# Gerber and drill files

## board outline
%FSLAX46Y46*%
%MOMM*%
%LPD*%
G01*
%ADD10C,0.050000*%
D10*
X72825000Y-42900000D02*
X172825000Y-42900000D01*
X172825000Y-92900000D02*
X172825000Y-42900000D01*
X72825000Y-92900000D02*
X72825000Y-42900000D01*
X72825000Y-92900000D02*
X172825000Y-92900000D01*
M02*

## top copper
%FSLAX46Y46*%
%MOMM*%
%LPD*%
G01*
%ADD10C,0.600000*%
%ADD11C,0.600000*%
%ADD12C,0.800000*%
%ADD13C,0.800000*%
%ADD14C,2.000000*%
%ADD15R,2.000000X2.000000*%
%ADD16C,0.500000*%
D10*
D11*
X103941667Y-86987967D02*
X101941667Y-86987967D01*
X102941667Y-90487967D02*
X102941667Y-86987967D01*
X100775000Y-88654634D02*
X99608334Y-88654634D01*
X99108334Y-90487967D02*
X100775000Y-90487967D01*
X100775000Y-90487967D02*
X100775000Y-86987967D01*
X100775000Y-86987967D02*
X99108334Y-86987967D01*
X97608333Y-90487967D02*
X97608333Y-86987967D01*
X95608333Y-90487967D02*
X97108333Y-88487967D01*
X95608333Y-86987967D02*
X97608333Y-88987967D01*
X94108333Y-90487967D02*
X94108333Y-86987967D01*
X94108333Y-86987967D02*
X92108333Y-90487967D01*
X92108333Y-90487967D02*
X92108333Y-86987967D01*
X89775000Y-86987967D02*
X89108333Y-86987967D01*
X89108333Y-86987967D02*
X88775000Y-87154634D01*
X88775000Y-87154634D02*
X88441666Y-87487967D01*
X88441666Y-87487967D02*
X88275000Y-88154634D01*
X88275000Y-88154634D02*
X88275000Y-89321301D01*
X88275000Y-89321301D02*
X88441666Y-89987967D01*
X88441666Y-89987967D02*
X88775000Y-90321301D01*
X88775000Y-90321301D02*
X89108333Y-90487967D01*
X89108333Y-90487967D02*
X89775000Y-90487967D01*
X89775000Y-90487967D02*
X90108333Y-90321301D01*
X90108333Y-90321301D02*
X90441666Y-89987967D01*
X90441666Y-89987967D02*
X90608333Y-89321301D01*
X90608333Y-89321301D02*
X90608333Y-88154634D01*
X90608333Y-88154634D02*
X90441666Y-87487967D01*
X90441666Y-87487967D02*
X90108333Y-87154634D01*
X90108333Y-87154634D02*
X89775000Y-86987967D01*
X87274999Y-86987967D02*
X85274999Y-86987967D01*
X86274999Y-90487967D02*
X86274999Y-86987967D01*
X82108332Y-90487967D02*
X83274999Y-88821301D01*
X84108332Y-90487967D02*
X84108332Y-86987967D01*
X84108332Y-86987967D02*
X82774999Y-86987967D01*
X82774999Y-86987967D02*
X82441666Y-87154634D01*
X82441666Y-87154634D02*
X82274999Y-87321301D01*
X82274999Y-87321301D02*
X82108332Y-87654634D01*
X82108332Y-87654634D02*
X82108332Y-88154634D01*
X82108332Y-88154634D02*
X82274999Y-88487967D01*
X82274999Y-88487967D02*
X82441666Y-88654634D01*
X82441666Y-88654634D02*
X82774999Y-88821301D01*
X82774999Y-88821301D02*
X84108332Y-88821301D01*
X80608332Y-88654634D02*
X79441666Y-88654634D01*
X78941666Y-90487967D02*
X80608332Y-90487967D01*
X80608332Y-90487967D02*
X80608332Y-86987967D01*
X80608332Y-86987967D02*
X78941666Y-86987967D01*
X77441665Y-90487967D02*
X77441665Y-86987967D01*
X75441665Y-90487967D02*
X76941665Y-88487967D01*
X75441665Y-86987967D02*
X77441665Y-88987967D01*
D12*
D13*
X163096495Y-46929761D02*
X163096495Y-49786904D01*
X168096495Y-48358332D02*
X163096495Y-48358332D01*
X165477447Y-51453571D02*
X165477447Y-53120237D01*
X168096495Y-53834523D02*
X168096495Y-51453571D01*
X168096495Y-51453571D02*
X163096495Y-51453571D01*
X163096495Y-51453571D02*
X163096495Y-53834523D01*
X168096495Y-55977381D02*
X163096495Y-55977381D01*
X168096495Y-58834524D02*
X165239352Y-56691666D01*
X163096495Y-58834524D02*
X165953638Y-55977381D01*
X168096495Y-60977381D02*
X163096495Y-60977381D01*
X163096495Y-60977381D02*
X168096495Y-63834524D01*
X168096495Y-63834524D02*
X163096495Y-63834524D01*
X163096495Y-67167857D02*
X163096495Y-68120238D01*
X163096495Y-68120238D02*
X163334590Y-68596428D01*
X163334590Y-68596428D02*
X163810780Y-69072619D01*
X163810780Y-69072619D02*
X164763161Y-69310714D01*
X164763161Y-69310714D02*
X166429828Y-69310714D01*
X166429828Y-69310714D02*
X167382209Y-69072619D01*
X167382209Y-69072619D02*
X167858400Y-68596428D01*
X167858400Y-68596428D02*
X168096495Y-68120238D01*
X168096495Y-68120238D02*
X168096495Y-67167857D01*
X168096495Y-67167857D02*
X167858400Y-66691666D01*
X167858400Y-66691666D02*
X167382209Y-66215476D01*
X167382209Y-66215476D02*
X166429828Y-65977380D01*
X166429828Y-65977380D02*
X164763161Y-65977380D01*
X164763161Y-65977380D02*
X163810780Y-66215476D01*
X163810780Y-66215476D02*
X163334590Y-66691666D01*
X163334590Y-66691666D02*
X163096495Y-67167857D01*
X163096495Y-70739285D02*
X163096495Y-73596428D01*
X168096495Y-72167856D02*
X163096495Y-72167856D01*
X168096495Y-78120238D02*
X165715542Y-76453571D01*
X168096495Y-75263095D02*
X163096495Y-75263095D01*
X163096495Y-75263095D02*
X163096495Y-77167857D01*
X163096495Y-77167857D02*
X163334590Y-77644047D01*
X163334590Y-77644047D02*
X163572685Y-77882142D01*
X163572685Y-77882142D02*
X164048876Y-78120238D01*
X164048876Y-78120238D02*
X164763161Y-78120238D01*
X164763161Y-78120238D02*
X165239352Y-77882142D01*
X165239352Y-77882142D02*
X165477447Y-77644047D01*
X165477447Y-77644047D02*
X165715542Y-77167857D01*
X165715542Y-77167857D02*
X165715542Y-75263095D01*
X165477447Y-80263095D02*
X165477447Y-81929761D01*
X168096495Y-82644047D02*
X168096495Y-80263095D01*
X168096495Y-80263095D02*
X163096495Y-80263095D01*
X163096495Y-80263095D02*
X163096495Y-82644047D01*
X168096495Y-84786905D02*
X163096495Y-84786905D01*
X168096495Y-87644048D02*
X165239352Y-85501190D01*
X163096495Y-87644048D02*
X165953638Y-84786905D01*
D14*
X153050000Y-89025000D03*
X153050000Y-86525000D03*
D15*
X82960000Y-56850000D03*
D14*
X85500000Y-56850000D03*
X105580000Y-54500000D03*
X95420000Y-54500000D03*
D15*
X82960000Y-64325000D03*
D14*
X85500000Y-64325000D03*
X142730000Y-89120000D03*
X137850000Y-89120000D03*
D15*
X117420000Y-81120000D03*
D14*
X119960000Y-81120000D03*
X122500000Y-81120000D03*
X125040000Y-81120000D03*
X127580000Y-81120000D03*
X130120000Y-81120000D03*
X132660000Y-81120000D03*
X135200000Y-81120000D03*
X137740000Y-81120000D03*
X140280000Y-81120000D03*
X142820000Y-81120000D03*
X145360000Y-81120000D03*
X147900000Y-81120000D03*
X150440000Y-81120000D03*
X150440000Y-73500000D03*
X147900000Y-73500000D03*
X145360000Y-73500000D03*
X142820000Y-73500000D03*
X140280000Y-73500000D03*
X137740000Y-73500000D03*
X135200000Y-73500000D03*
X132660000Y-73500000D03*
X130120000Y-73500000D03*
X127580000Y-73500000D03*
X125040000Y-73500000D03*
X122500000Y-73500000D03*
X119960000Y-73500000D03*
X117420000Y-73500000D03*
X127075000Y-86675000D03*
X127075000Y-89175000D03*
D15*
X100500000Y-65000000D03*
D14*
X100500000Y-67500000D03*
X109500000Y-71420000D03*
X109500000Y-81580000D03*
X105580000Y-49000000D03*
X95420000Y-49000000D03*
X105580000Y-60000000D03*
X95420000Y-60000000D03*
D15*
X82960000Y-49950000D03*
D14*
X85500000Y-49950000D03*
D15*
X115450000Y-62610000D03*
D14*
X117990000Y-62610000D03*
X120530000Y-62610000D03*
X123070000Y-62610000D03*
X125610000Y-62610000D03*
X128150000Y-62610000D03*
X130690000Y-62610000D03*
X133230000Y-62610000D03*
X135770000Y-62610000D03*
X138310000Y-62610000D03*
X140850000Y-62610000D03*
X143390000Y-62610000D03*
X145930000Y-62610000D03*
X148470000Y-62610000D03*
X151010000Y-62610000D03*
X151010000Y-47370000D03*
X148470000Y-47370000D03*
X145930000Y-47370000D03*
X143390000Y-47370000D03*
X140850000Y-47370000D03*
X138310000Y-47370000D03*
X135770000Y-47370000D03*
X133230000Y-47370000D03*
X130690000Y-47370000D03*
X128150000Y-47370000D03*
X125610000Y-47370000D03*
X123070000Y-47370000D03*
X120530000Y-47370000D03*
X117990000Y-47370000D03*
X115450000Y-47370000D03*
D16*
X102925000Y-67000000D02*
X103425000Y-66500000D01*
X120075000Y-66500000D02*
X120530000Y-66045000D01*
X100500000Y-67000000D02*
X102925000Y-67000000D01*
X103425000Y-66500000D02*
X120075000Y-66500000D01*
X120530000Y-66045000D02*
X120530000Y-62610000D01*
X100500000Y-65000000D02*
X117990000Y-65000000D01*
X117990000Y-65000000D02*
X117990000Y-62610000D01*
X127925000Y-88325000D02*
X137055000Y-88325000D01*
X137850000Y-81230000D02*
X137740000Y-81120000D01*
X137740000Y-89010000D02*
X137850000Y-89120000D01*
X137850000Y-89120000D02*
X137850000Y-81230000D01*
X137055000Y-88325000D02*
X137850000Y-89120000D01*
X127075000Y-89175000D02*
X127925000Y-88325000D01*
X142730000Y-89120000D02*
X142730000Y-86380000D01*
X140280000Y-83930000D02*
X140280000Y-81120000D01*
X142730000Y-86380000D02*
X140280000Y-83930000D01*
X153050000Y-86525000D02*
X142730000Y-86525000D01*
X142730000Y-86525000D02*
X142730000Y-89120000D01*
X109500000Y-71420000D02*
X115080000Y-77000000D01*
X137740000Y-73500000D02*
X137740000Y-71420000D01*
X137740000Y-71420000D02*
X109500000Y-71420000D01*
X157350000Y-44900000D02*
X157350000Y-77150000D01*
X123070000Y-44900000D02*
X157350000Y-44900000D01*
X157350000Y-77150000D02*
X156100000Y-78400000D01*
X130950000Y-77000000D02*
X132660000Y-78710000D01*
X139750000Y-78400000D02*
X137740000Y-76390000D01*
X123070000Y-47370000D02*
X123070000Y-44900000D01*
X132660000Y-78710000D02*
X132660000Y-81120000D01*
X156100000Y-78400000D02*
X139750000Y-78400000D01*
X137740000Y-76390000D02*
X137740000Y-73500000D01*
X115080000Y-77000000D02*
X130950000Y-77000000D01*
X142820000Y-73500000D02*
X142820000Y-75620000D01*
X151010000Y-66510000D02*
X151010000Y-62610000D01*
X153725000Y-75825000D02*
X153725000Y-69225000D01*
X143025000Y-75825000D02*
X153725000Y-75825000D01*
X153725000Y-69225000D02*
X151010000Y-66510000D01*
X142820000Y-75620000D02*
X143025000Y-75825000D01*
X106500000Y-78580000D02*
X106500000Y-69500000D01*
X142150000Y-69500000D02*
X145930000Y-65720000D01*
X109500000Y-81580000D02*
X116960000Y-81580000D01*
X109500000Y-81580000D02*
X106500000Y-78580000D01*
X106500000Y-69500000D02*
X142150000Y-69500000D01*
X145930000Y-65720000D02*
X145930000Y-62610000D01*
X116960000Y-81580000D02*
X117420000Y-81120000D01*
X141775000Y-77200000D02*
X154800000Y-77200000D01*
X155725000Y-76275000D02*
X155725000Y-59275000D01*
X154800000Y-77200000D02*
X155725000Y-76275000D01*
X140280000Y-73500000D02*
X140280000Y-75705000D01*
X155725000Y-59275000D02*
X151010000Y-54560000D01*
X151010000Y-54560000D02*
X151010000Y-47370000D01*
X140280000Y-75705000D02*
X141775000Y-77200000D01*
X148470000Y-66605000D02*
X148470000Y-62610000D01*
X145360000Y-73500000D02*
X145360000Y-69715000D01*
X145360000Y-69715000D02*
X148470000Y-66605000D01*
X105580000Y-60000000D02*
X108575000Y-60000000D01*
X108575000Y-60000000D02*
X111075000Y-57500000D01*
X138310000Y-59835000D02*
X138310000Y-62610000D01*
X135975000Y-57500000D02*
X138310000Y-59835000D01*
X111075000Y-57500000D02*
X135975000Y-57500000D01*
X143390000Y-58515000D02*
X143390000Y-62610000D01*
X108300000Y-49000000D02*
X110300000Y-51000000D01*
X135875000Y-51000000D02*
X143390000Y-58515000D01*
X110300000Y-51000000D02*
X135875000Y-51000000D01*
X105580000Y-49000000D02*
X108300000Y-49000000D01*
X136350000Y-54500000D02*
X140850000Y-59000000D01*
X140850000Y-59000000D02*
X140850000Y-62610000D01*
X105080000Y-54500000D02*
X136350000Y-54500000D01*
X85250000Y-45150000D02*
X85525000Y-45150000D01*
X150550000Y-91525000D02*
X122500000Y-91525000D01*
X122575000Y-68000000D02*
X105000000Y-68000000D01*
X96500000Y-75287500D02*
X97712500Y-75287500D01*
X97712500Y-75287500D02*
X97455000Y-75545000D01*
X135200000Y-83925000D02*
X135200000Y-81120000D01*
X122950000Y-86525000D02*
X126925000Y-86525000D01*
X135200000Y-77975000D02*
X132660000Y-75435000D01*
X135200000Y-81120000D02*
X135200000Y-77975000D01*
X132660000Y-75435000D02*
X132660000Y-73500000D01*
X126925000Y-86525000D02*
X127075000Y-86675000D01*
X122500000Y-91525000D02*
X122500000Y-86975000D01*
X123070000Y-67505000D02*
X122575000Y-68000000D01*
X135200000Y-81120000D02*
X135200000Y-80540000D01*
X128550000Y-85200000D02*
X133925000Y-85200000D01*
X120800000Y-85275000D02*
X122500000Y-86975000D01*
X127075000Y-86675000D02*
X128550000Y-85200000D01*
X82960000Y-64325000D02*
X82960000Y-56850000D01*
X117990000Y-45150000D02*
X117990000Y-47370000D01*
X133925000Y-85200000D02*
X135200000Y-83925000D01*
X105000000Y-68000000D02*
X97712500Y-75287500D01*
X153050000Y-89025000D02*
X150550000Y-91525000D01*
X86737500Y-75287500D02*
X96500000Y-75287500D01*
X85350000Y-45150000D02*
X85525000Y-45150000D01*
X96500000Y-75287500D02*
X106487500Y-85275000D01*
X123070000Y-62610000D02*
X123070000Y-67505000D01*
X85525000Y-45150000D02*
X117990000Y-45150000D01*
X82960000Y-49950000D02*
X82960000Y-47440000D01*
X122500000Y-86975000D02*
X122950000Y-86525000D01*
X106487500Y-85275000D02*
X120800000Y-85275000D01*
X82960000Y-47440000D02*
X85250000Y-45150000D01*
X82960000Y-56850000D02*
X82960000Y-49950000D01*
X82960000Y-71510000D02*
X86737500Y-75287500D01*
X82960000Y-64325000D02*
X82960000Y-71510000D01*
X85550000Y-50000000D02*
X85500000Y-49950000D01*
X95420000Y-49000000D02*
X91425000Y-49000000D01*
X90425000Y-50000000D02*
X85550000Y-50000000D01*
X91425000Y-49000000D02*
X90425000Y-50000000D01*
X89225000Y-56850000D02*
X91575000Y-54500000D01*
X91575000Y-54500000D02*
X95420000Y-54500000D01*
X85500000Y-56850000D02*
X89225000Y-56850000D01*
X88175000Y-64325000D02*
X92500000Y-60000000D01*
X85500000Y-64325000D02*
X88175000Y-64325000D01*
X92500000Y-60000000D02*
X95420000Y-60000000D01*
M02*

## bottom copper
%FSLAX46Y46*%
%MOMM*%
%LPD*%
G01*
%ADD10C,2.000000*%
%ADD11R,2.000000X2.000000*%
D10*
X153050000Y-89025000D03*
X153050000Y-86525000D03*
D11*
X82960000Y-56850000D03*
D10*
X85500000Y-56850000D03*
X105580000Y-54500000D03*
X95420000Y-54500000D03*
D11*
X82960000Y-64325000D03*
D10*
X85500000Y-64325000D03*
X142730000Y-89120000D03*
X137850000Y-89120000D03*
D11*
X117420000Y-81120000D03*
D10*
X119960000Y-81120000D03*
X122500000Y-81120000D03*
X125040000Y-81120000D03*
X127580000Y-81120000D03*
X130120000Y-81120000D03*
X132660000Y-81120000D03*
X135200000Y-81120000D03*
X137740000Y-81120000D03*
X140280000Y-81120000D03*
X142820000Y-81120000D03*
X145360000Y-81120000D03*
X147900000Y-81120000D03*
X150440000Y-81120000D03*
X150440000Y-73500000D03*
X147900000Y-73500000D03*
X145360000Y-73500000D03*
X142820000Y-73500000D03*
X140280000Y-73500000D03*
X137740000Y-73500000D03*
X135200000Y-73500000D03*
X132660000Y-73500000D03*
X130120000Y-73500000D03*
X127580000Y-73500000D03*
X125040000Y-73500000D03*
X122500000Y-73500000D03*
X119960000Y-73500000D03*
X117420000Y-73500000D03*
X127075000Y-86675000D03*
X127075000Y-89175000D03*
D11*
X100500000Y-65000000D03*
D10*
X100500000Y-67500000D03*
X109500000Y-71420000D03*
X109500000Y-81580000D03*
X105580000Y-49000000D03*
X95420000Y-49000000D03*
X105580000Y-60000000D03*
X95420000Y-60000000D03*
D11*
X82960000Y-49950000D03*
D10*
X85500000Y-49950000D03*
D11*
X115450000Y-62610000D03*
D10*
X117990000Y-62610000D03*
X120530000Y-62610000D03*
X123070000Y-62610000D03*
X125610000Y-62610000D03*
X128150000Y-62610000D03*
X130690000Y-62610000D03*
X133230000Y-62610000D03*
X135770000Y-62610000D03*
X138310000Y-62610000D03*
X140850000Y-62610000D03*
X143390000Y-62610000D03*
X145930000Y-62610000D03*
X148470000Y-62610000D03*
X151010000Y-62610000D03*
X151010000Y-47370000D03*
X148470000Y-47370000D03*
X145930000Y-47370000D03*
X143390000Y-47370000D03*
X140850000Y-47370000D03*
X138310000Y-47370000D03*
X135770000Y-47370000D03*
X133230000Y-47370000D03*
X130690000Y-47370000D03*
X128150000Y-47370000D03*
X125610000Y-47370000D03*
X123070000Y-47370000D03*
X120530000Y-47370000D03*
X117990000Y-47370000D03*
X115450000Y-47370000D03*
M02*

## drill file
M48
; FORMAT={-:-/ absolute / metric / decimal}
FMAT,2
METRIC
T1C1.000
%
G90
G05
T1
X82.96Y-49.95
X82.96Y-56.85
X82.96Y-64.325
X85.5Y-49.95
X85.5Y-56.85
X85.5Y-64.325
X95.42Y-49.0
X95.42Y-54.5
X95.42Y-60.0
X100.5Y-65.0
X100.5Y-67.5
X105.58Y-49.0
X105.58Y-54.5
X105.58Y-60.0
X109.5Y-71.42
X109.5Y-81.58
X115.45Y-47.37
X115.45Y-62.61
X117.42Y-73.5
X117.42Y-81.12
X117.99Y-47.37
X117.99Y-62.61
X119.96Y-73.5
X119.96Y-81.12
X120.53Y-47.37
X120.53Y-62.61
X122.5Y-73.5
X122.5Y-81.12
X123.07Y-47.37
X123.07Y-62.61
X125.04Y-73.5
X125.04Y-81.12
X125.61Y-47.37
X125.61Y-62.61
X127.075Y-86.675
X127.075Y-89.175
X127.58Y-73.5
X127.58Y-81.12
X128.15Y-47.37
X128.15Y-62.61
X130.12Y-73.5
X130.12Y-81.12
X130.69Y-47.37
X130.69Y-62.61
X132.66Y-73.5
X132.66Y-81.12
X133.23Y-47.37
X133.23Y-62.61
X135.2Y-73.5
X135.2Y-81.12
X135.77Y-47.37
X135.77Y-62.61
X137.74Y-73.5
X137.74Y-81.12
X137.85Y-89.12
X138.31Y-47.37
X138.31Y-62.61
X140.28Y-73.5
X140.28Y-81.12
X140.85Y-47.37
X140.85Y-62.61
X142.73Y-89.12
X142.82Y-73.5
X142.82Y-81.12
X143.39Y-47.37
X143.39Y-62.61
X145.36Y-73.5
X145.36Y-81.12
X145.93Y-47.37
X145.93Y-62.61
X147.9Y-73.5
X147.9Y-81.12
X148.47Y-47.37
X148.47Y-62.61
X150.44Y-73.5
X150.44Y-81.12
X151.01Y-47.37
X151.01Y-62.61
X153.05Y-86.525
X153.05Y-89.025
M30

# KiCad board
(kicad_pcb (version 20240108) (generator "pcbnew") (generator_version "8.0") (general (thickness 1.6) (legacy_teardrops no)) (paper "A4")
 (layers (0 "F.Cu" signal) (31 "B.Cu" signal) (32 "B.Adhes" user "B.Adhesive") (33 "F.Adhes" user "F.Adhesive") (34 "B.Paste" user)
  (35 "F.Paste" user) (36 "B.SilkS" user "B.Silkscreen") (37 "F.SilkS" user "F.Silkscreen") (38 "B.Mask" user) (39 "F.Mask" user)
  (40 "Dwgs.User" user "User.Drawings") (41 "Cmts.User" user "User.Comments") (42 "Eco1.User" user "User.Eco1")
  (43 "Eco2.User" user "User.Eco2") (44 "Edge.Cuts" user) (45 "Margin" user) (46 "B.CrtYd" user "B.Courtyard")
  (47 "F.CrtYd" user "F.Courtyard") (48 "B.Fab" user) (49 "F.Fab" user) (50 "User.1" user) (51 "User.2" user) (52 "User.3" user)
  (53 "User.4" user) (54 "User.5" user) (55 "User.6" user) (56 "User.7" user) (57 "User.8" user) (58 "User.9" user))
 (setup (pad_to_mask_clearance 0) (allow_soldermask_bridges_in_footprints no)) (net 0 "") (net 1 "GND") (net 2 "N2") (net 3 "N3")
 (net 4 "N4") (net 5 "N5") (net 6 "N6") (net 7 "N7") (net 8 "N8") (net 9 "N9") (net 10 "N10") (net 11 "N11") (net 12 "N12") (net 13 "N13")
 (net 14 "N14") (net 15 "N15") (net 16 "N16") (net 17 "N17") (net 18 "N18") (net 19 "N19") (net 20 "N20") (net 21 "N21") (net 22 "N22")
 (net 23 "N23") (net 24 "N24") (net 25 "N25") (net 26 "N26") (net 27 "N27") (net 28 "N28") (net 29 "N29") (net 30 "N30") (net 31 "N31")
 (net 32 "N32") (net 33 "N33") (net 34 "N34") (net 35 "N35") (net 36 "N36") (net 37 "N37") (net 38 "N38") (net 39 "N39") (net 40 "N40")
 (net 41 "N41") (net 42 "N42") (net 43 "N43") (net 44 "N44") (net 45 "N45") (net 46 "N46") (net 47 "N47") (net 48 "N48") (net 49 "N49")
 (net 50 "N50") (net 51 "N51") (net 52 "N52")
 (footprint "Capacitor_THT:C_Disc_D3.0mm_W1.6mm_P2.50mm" (layer "F.Cu") (at 153.05 89.025 90)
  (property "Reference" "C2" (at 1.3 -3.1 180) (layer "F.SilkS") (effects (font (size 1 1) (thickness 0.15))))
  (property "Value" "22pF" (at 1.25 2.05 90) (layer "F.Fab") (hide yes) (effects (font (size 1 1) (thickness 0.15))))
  (pad "1" thru_hole circle (at 0 0 90) (size 2 2) (drill 1) (layers "*.Cu" "*.Mask") (remove_unused_layers no) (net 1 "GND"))
  (pad "2" thru_hole circle (at 2.5 0 90) (size 2 2) (drill 1) (layers "*.Cu" "*.Mask") (remove_unused_layers no) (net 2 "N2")))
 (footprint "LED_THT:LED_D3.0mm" (layer "F.Cu") (at 82.96 56.85)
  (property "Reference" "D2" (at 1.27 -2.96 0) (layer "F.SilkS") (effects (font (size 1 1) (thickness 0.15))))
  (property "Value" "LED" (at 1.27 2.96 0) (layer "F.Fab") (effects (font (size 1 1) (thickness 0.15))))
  (pad "1" thru_hole rect (at 0 0) (size 2 2) (drill 1) (layers "*.Cu" "*.Mask") (remove_unused_layers no) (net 1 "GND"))
  (pad "2" thru_hole circle (at 2.54 0) (size 2 2) (drill 1) (layers "*.Cu" "*.Mask") (remove_unused_layers no) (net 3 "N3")))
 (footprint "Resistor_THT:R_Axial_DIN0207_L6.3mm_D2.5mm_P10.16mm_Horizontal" (layer "F.Cu") (at 105.58 54.5 180)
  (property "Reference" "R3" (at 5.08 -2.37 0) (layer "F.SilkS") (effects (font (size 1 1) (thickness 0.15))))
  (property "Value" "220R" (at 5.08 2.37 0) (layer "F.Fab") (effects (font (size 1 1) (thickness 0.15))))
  (pad "1" thru_hole circle (at 0 0 180) (size 2 2) (drill 1) (layers "*.Cu" "*.Mask") (remove_unused_layers no) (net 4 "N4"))
  (pad "2" thru_hole circle (at 10.16 0 180) (size 2 2) (drill 1) (layers "*.Cu" "*.Mask") (remove_unused_layers no) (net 3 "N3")))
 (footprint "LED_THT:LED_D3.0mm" (layer "F.Cu") (at 82.96 64.325)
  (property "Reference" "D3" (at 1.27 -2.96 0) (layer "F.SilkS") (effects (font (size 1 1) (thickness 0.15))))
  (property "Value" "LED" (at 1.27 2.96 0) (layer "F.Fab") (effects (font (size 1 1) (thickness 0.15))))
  (pad "1" thru_hole rect (at 0 0) (size 2 2) (drill 1) (layers "*.Cu" "*.Mask") (remove_unused_layers no) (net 1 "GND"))
  (pad "2" thru_hole circle (at 2.54 0) (size 2 2) (drill 1) (layers "*.Cu" "*.Mask") (remove_unused_layers no) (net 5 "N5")))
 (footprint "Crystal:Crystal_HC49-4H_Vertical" (layer "F.Cu") (at 142.73 89.12 180)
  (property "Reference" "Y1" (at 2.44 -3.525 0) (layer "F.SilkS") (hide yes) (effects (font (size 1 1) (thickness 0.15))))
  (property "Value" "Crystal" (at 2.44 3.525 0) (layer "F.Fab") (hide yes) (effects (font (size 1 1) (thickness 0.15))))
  (pad "1" thru_hole circle (at 0 0 180) (size 2 2) (drill 1) (layers "*.Cu" "*.Mask") (remove_unused_layers no) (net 2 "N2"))
  (pad "2" thru_hole circle (at 4.88 0 180) (size 2 2) (drill 1) (layers "*.Cu" "*.Mask") (remove_unused_layers no) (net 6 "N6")))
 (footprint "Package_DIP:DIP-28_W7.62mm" (layer "F.Cu") (at 117.42 81.12 90)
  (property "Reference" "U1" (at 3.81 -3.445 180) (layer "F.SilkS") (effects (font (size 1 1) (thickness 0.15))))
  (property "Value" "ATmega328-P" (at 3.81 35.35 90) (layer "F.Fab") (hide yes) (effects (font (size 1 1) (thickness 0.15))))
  (pad "1" thru_hole rect (at 0 0 90) (size 2 2) (drill 1) (layers "*.Cu" "*.Mask") (remove_unused_layers no) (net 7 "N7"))
  (pad "2" thru_hole circle (at 0 2.54 90) (size 2 2) (drill 1) (layers "*.Cu" "*.Mask") (remove_unused_layers no) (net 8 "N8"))
  (pad "3" thru_hole circle (at 0 5.08 90) (size 2 2) (drill 1) (layers "*.Cu" "*.Mask") (remove_unused_layers no) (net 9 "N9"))
  (pad "4" thru_hole circle (at 0 7.62 90) (size 2 2) (drill 1) (layers "*.Cu" "*.Mask") (remove_unused_layers no) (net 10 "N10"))
  (pad "5" thru_hole circle (at 0 10.16 90) (size 2 2) (drill 1) (layers "*.Cu" "*.Mask") (remove_unused_layers no) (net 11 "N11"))
  (pad "6" thru_hole circle (at 0 12.7 90) (size 2 2) (drill 1) (layers "*.Cu" "*.Mask") (remove_unused_layers no) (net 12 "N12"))
  (pad "7" thru_hole circle (at 0 15.24 90) (size 2 2) (drill 1) (layers "*.Cu" "*.Mask") (remove_unused_layers no) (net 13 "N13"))
  (pad "8" thru_hole circle (at 0 17.78 90) (size 2 2) (drill 1) (layers "*.Cu" "*.Mask") (remove_unused_layers no) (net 1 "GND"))
  (pad "9" thru_hole circle (at 0 20.32 90) (size 2 2) (drill 1) (layers "*.Cu" "*.Mask") (remove_unused_layers no) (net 6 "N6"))
  (pad "10" thru_hole circle (at 0 22.86 90) (size 2 2) (drill 1) (layers "*.Cu" "*.Mask") (remove_unused_layers no) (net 2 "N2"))
  (pad "11" thru_hole circle (at 0 25.4 90) (size 2 2) (drill 1) (layers "*.Cu" "*.Mask") (remove_unused_layers no) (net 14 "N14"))
  (pad "12" thru_hole circle (at 0 27.94 90) (size 2 2) (drill 1) (layers "*.Cu" "*.Mask") (remove_unused_layers no) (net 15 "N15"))
  (pad "13" thru_hole circle (at 0 30.48 90) (size 2 2) (drill 1) (layers "*.Cu" "*.Mask") (remove_unused_layers no) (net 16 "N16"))
  (pad "14" thru_hole circle (at 0 33.02 90) (size 2 2) (drill 1) (layers "*.Cu" "*.Mask") (remove_unused_layers no) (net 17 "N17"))
  (pad "15" thru_hole circle (at 7.62 33.02 90) (size 2 2) (drill 1) (layers "*.Cu" "*.Mask") (remove_unused_layers no) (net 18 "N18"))
  (pad "16" thru_hole circle (at 7.62 30.48 90) (size 2 2) (drill 1) (layers "*.Cu" "*.Mask") (remove_unused_layers no) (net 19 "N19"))
  (pad "17" thru_hole circle (at 7.62 27.94 90) (size 2 2) (drill 1) (layers "*.Cu" "*.Mask") (remove_unused_layers no) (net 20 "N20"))
  (pad "18" thru_hole circle (at 7.62 25.4 90) (size 2 2) (drill 1) (layers "*.Cu" "*.Mask") (remove_unused_layers no) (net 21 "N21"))
  (pad "19" thru_hole circle (at 7.62 22.86 90) (size 2 2) (drill 1) (layers "*.Cu" "*.Mask") (remove_unused_layers no) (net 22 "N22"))
  (pad "20" thru_hole circle (at 7.62 20.32 90) (size 2 2) (drill 1) (layers "*.Cu" "*.Mask") (remove_unused_layers no) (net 13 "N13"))
  (pad "21" thru_hole circle (at 7.62 17.78 90) (size 2 2) (drill 1) (layers "*.Cu" "*.Mask") (remove_unused_layers no) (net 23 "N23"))
  (pad "22" thru_hole circle (at 7.62 15.24 90) (size 2 2) (drill 1) (layers "*.Cu" "*.Mask") (remove_unused_layers no) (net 1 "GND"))
  (pad "23" thru_hole circle (at 7.62 12.7 90) (size 2 2) (drill 1) (layers "*.Cu" "*.Mask") (remove_unused_layers no) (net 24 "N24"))
  (pad "24" thru_hole circle (at 7.62 10.16 90) (size 2 2) (drill 1) (layers "*.Cu" "*.Mask") (remove_unused_layers no) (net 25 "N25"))
  (pad "25" thru_hole circle (at 7.62 7.62 90) (size 2 2) (drill 1) (layers "*.Cu" "*.Mask") (remove_unused_layers no) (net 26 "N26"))
  (pad "26" thru_hole circle (at 7.62 5.08 90) (size 2 2) (drill 1) (layers "*.Cu" "*.Mask") (remove_unused_layers no) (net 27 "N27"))
  (pad "27" thru_hole circle (at 7.62 2.54 90) (size 2 2) (drill 1) (layers "*.Cu" "*.Mask") (remove_unused_layers no) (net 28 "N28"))
  (pad "28" thru_hole circle (at 7.62 0 90) (size 2 2) (drill 1) (layers "*.Cu" "*.Mask") (remove_unused_layers no) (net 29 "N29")))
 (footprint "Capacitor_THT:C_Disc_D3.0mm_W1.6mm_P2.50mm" (layer "F.Cu") (at 127.075 86.675 -90)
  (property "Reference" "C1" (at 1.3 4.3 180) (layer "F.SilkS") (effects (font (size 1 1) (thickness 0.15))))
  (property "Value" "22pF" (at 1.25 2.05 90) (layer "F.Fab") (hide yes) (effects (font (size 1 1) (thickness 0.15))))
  (pad "1" thru_hole circle (at 0 0 270) (size 2 2) (drill 1) (layers "*.Cu" "*.Mask") (remove_unused_layers no) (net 1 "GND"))
  (pad "2" thru_hole circle (at 2.5 0 270) (size 2 2) (drill 1) (layers "*.Cu" "*.Mask") (remove_unused_layers no) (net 6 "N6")))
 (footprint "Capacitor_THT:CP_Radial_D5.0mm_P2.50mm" (layer "F.Cu") (at 100.5 65 -90)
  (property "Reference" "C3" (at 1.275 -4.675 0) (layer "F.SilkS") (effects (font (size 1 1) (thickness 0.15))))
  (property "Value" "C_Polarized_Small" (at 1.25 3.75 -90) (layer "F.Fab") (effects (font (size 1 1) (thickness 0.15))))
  (pad "1" thru_hole rect (at 0 0 270) (size 2 2) (drill 1) (layers "*.Cu" "*.Mask") (remove_unused_layers no) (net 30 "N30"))
  (pad "2" thru_hole circle (at 2.5 0 270) (size 2 2) (drill 1) (layers "*.Cu" "*.Mask") (remove_unused_layers no) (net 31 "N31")))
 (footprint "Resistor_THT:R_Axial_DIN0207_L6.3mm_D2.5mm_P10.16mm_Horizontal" (layer "F.Cu") (at 109.5 71.42 -90)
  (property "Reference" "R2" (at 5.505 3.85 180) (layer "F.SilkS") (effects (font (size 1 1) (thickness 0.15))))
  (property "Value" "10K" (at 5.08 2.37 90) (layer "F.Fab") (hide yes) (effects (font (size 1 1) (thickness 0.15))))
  (pad "1" thru_hole circle (at 0 0 270) (size 2 2) (drill 1) (layers "*.Cu" "*.Mask") (remove_unused_layers no) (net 13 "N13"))
  (pad "2" thru_hole circle (at 10.16 0 270) (size 2 2) (drill 1) (layers "*.Cu" "*.Mask") (remove_unused_layers no) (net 7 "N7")))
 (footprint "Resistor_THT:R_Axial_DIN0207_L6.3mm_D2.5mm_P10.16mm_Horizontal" (layer "F.Cu") (at 105.58 49 180)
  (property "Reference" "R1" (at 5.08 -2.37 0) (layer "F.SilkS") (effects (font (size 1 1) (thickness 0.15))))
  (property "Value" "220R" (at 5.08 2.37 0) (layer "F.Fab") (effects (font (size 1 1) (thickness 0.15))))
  (pad "1" thru_hole circle (at 0 0 180) (size 2 2) (drill 1) (layers "*.Cu" "*.Mask") (remove_unused_layers no) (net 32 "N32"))
  (pad "2" thru_hole circle (at 10.16 0 180) (size 2 2) (drill 1) (layers "*.Cu" "*.Mask") (remove_unused_layers no) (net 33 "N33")))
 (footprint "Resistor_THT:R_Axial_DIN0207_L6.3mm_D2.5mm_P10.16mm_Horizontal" (layer "F.Cu") (at 105.58 60 180)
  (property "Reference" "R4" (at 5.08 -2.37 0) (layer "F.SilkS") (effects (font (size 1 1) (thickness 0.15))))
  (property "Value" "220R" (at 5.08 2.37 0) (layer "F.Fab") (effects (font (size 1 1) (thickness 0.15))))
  (pad "1" thru_hole circle (at 0 0 180) (size 2 2) (drill 1) (layers "*.Cu" "*.Mask") (remove_unused_layers no) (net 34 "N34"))
  (pad "2" thru_hole circle (at 10.16 0 180) (size 2 2) (drill 1) (layers "*.Cu" "*.Mask") (remove_unused_layers no) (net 5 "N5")))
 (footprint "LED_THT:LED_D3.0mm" (layer "F.Cu") (at 82.96 49.95)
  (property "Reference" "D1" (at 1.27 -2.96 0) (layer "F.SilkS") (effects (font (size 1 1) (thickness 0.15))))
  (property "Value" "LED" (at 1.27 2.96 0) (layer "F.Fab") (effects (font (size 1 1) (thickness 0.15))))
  (pad "1" thru_hole rect (at 0 0) (size 2 2) (drill 1) (layers "*.Cu" "*.Mask") (remove_unused_layers no) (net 1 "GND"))
  (pad "2" thru_hole circle (at 2.54 0) (size 2 2) (drill 1) (layers "*.Cu" "*.Mask") (remove_unused_layers no) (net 33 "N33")))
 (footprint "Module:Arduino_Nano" (layer "F.Cu") (at 115.45 62.61 90)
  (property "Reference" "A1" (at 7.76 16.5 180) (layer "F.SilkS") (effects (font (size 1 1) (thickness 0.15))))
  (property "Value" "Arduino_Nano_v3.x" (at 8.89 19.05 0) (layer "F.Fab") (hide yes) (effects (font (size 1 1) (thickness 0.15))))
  (pad "1" thru_hole rect (at 0 0 90) (size 2 2) (drill 1) (layers "*.Cu" "*.Mask") (remove_unused_layers no) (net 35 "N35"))
  (pad "2" thru_hole circle (at 0 2.54 90) (size 2 2) (drill 1) (layers "*.Cu" "*.Mask") (remove_unused_layers no) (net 30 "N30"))
  (pad "3" thru_hole circle (at 0 5.08 90) (size 2 2) (drill 1) (layers "*.Cu" "*.Mask") (remove_unused_layers no) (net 31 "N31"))
  (pad "4" thru_hole circle (at 0 7.62 90) (size 2 2) (drill 1) (layers "*.Cu" "*.Mask") (remove_unused_layers no) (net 1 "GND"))
  (pad "5" thru_hole circle (at 0 10.16 90) (size 2 2) (drill 1) (layers "*.Cu" "*.Mask") (remove_unused_layers no) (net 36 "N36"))
  (pad "6" thru_hole circle (at 0 12.7 90) (size 2 2) (drill 1) (layers "*.Cu" "*.Mask") (remove_unused_layers no) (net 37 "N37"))
  (pad "7" thru_hole circle (at 0 15.24 90) (size 2 2) (drill 1) (layers "*.Cu" "*.Mask") (remove_unused_layers no) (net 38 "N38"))
  (pad "8" thru_hole circle (at 0 17.78 90) (size 2 2) (drill 1) (layers "*.Cu" "*.Mask") (remove_unused_layers no) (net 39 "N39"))
  (pad "9" thru_hole circle (at 0 20.32 90) (size 2 2) (drill 1) (layers "*.Cu" "*.Mask") (remove_unused_layers no) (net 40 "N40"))
  (pad "10" thru_hole circle (at 0 22.86 90) (size 2 2) (drill 1) (layers "*.Cu" "*.Mask") (remove_unused_layers no) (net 34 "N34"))
  (pad "11" thru_hole circle (at 0 25.4 90) (size 2 2) (drill 1) (layers "*.Cu" "*.Mask") (remove_unused_layers no) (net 4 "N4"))
  (pad "12" thru_hole circle (at 0 27.94 90) (size 2 2) (drill 1) (layers "*.Cu" "*.Mask") (remove_unused_layers no) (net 32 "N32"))
  (pad "13" thru_hole circle (at 0 30.48 90) (size 2 2) (drill 1) (layers "*.Cu" "*.Mask") (remove_unused_layers no) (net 7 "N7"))
  (pad "14" thru_hole circle (at 0 33.02 90) (size 2 2) (drill 1) (layers "*.Cu" "*.Mask") (remove_unused_layers no) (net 20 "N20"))
  (pad "15" thru_hole circle (at 0 35.56 90) (size 2 2) (drill 1) (layers "*.Cu" "*.Mask") (remove_unused_layers no) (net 21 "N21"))
  (pad "16" thru_hole circle (at 15.24 35.56 90) (size 2 2) (drill 1) (layers "*.Cu" "*.Mask") (remove_unused_layers no) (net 22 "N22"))
  (pad "17" thru_hole circle (at 15.24 33.02 90) (size 2 2) (drill 1) (layers "*.Cu" "*.Mask") (remove_unused_layers no) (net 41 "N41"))
  (pad "18" thru_hole circle (at 15.24 30.48 90) (size 2 2) (drill 1) (layers "*.Cu" "*.Mask") (remove_unused_layers no) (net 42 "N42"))
  (pad "19" thru_hole circle (at 15.24 27.94 90) (size 2 2) (drill 1) (layers "*.Cu" "*.Mask") (remove_unused_layers no) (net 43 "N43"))
  (pad "20" thru_hole circle (at 15.24 25.4 90) (size 2 2) (drill 1) (layers "*.Cu" "*.Mask") (remove_unused_layers no) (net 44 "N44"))
  (pad "21" thru_hole circle (at 15.24 22.86 90) (size 2 2) (drill 1) (layers "*.Cu" "*.Mask") (remove_unused_layers no) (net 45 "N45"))
  (pad "22" thru_hole circle (at 15.24 20.32 90) (size 2 2) (drill 1) (layers "*.Cu" "*.Mask") (remove_unused_layers no) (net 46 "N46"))
  (pad "23" thru_hole circle (at 15.24 17.78 90) (size 2 2) (drill 1) (layers "*.Cu" "*.Mask") (remove_unused_layers no) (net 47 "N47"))
  (pad "24" thru_hole circle (at 15.24 15.24 90) (size 2 2) (drill 1) (layers "*.Cu" "*.Mask") (remove_unused_layers no) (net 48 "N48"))
  (pad "25" thru_hole circle (at 15.24 12.7 90) (size 2 2) (drill 1) (layers "*.Cu" "*.Mask") (remove_unused_layers no) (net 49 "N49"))
  (pad "26" thru_hole circle (at 15.24 10.16 90) (size 2 2) (drill 1) (layers "*.Cu" "*.Mask") (remove_unused_layers no) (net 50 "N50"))
  (pad "27" thru_hole circle (at 15.24 7.62 90) (size 2 2) (drill 1) (layers "*.Cu" "*.Mask") (remove_unused_layers no) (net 13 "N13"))
  (pad "28" thru_hole circle (at 15.24 5.08 90) (size 2 2) (drill 1) (layers "*.Cu" "*.Mask") (remove_unused_layers no) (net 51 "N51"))
  (pad "29" thru_hole circle (at 15.24 2.54 90) (size 2 2) (drill 1) (layers "*.Cu" "*.Mask") (remove_unused_layers no) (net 1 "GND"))
  (pad "30" thru_hole circle (at 15.24 0 90) (size 2 2) (drill 1) (layers "*.Cu" "*.Mask") (remove_unused_layers no) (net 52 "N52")))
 (gr_line (start 72.825 42.9) (end 172.825 42.9) (stroke (width 0.05) (type default)) (layer "Edge.Cuts"))
 (gr_line (start 172.825 92.9) (end 172.825 42.9) (stroke (width 0.05) (type default)) (layer "Edge.Cuts"))
 (gr_line (start 72.825 92.9) (end 72.825 42.9) (stroke (width 0.05) (type default)) (layer "Edge.Cuts"))
 (gr_line (start 72.825 92.9) (end 172.825 92.9) (stroke (width 0.05) (type default)) (layer "Edge.Cuts"))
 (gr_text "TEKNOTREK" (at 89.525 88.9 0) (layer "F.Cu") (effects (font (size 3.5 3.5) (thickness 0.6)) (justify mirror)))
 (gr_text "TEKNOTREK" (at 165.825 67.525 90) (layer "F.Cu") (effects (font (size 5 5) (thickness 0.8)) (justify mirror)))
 (segment (start 102.925 67) (end 103.425 66.5) (width 0.5) (layer "F.Cu") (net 31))
 (segment (start 120.075 66.5) (end 120.53 66.045) (width 0.5) (layer "F.Cu") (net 31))
 (segment (start 100.5 67) (end 102.925 67) (width 0.5) (layer "F.Cu") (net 31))
 (segment (start 103.425 66.5) (end 120.075 66.5) (width 0.5) (layer "F.Cu") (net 31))
 (segment (start 120.53 66.045) (end 120.53 62.61) (width 0.5) (layer "F.Cu") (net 31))
 (segment (start 100.5 65) (end 117.99 65) (width 0.5) (layer "F.Cu") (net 30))
 (segment (start 117.99 65) (end 117.99 62.61) (width 0.5) (layer "F.Cu") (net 30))
 (segment (start 127.925 88.325) (end 137.055 88.325) (width 0.5) (layer "F.Cu") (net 6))
 (segment (start 137.85 81.23) (end 137.74 81.12) (width 0.5) (layer "F.Cu") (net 6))
 (segment (start 137.74 89.01) (end 137.85 89.12) (width 0.5) (layer "F.Cu") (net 6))
 (segment (start 137.85 89.12) (end 137.85 81.23) (width 0.5) (layer "F.Cu") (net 6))
 (segment (start 137.055 88.325) (end 137.85 89.12) (width 0.5) (layer "F.Cu") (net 6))
 (segment (start 127.075 89.175) (end 127.925 88.325) (width 0.5) (layer "F.Cu") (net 6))
 (segment (start 142.73 89.12) (end 142.73 86.38) (width 0.5) (layer "F.Cu") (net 2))
 (segment (start 140.28 83.93) (end 140.28 81.12) (width 0.5) (layer "F.Cu") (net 2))
 (segment (start 142.73 86.38) (end 140.28 83.93) (width 0.5) (layer "F.Cu") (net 2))
 (segment (start 153.05 86.525) (end 142.73 86.525) (width 0.5) (layer "F.Cu") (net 2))
 (segment (start 142.73 86.525) (end 142.73 89.12) (width 0.5) (layer "F.Cu") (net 2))
 (segment (start 109.5 71.42) (end 115.08 77) (width 0.5) (layer "F.Cu") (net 13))
 (segment (start 137.74 73.5) (end 137.74 71.42) (width 0.5) (layer "F.Cu") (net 13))
 (segment (start 137.74 71.42) (end 109.5 71.42) (width 0.5) (layer "F.Cu") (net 13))
 (segment (start 157.35 44.9) (end 157.35 77.15) (width 0.5) (layer "F.Cu") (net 13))
 (segment (start 123.07 44.9) (end 157.35 44.9) (width 0.5) (layer "F.Cu") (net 13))
 (segment (start 157.35 77.15) (end 156.1 78.4) (width 0.5) (layer "F.Cu") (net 13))
 (segment (start 130.95 77) (end 132.66 78.71) (width 0.5) (layer "F.Cu") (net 13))
 (segment (start 139.75 78.4) (end 137.74 76.39) (width 0.5) (layer "F.Cu") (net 13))
 (segment (start 123.07 47.37) (end 123.07 44.9) (width 0.5) (layer "F.Cu") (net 13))
 (segment (start 132.66 78.71) (end 132.66 81.12) (width 0.5) (layer "F.Cu") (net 13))
 (segment (start 156.1 78.4) (end 139.75 78.4) (width 0.5) (layer "F.Cu") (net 13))
 (segment (start 137.74 76.39) (end 137.74 73.5) (width 0.5) (layer "F.Cu") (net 13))
 (segment (start 115.08 77) (end 130.95 77) (width 0.5) (layer "F.Cu") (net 13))
 (segment (start 142.82 73.5) (end 142.82 75.62) (width 0.5) (layer "F.Cu") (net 21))
 (segment (start 151.01 66.51) (end 151.01 62.61) (width 0.5) (layer "F.Cu") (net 21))
 (segment (start 153.725 75.825) (end 153.725 69.225) (width 0.5) (layer "F.Cu") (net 21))
 (segment (start 143.025 75.825) (end 153.725 75.825) (width 0.5) (layer "F.Cu") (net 21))
 (segment (start 153.725 69.225) (end 151.01 66.51) (width 0.5) (layer "F.Cu") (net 21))
 (segment (start 142.82 75.62) (end 143.025 75.825) (width 0.5) (layer "F.Cu") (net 21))
 (segment (start 106.5 78.58) (end 106.5 69.5) (width 0.5) (layer "F.Cu") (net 7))
 (segment (start 142.15 69.5) (end 145.93 65.72) (width 0.5) (layer "F.Cu") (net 7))
 (segment (start 109.5 81.58) (end 116.96 81.58) (width 0.5) (layer "F.Cu") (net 7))
 (segment (start 109.5 81.58) (end 106.5 78.58) (width 0.5) (layer "F.Cu") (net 7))
 (segment (start 106.5 69.5) (end 142.15 69.5) (width 0.5) (layer "F.Cu") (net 7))
 (segment (start 145.93 65.72) (end 145.93 62.61) (width 0.5) (layer "F.Cu") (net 7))
 (segment (start 116.96 81.58) (end 117.42 81.12) (width 0.5) (layer "F.Cu") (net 7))
 (segment (start 141.775 77.2) (end 154.8 77.2) (width 0.5) (layer "F.Cu") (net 22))
 (segment (start 155.725 76.275) (end 155.725 59.275) (width 0.5) (layer "F.Cu") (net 22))
 (segment (start 154.8 77.2) (end 155.725 76.275) (width 0.5) (layer "F.Cu") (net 22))
 (segment (start 140.28 73.5) (end 140.28 75.705) (width 0.5) (layer "F.Cu") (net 22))
 (segment (start 155.725 59.275) (end 151.01 54.56) (width 0.5) (layer "F.Cu") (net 22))
 (segment (start 151.01 54.56) (end 151.01 47.37) (width 0.5) (layer "F.Cu") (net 22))
 (segment (start 140.28 75.705) (end 141.775 77.2) (width 0.5) (layer "F.Cu") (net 22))
 (segment (start 148.47 66.605) (end 148.47 62.61) (width 0.5) (layer "F.Cu") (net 20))
 (segment (start 145.36 73.5) (end 145.36 69.715) (width 0.5) (layer "F.Cu") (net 20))
 (segment (start 145.36 69.715) (end 148.47 66.605) (width 0.5) (layer "F.Cu") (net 20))
 (segment (start 105.58 60) (end 108.575 60) (width 0.5) (layer "F.Cu") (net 34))
 (segment (start 108.575 60) (end 111.075 57.5) (width 0.5) (layer "F.Cu") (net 34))
 (segment (start 138.31 59.835) (end 138.31 62.61) (width 0.5) (layer "F.Cu") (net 34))
 (segment (start 135.975 57.5) (end 138.31 59.835) (width 0.5) (layer "F.Cu") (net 34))
 (segment (start 111.075 57.5) (end 135.975 57.5) (width 0.5) (layer "F.Cu") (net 34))
 (segment (start 143.39 58.515) (end 143.39 62.61) (width 0.5) (layer "F.Cu") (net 32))
 (segment (start 108.3 49) (end 110.3 51) (width 0.5) (layer "F.Cu") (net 32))
 (segment (start 135.875 51) (end 143.39 58.515) (width 0.5) (layer "F.Cu") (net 32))
 (segment (start 110.3 51) (end 135.875 51) (width 0.5) (layer "F.Cu") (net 32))
 (segment (start 105.58 49) (end 108.3 49) (width 0.5) (layer "F.Cu") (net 32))
 (segment (start 136.35 54.5) (end 140.85 59) (width 0.5) (layer "F.Cu") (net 4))
 (segment (start 140.85 59) (end 140.85 62.61) (width 0.5) (layer "F.Cu") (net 4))
 (segment (start 105.08 54.5) (end 136.35 54.5) (width 0.5) (layer "F.Cu") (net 4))
 (segment (start 85.25 45.15) (end 85.525 45.15) (width 0.5) (layer "F.Cu") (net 1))
 (segment (start 150.55 91.525) (end 122.5 91.525) (width 0.5) (layer "F.Cu") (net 1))
 (segment (start 122.575 68) (end 105 68) (width 0.5) (layer "F.Cu") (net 1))
 (segment (start 96.5 75.2875) (end 97.7125 75.2875) (width 0.5) (layer "F.Cu") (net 1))
 (segment (start 97.7125 75.2875) (end 97.455 75.545) (width 0.5) (layer "F.Cu") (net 1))
 (segment (start 135.2 83.925) (end 135.2 81.12) (width 0.5) (layer "F.Cu") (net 1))
 (segment (start 122.95 86.525) (end 126.925 86.525) (width 0.5) (layer "F.Cu") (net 1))
 (segment (start 135.2 77.975) (end 132.66 75.435) (width 0.5) (layer "F.Cu") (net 1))
 (segment (start 135.2 81.12) (end 135.2 77.975) (width 0.5) (layer "F.Cu") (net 1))
 (segment (start 132.66 75.435) (end 132.66 73.5) (width 0.5) (layer "F.Cu") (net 1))
 (segment (start 126.925 86.525) (end 127.075 86.675) (width 0.5) (layer "F.Cu") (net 1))
 (segment (start 122.5 91.525) (end 122.5 86.975) (width 0.5) (layer "F.Cu") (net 1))
 (segment (start 123.07 67.505) (end 122.575 68) (width 0.5) (layer "F.Cu") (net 1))
 (segment (start 135.2 81.12) (end 135.2 80.54) (width 0.5) (layer "F.Cu") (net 1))
 (segment (start 128.55 85.2) (end 133.925 85.2) (width 0.5) (layer "F.Cu") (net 1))
 (segment (start 120.8 85.275) (end 122.5 86.975) (width 0.5) (layer "F.Cu") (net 1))
 (segment (start 127.075 86.675) (end 128.55 85.2) (width 0.5) (layer "F.Cu") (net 1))
 (segment (start 82.96 64.325) (end 82.96 56.85) (width 0.5) (layer "F.Cu") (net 1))
 (segment (start 117.99 45.15) (end 117.99 47.37) (width 0.5) (layer "F.Cu") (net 1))
 (segment (start 133.925 85.2) (end 135.2 83.925) (width 0.5) (layer "F.Cu") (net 1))
 (segment (start 105 68) (end 97.7125 75.2875) (width 0.5) (layer "F.Cu") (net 1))
 (segment (start 153.05 89.025) (end 150.55 91.525) (width 0.5) (layer "F.Cu") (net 1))
 (segment (start 86.7375 75.2875) (end 96.5 75.2875) (width 0.5) (layer "F.Cu") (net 1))
 (segment (start 85.35 45.15) (end 85.525 45.15) (width 0.5) (layer "F.Cu") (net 1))
 (segment (start 96.5 75.2875) (end 106.4875 85.275) (width 0.5) (layer "F.Cu") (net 1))
 (segment (start 123.07 62.61) (end 123.07 67.505) (width 0.5) (layer "F.Cu") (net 1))
 (segment (start 85.525 45.15) (end 117.99 45.15) (width 0.5) (layer "F.Cu") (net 1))
 (segment (start 82.96 49.95) (end 82.96 47.44) (width 0.5) (layer "F.Cu") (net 1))
 (segment (start 122.5 86.975) (end 122.95 86.525) (width 0.5) (layer "F.Cu") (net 1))
 (segment (start 106.4875 85.275) (end 120.8 85.275) (width 0.5) (layer "F.Cu") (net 1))
 (segment (start 82.96 47.44) (end 85.25 45.15) (width 0.5) (layer "F.Cu") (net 1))
 (segment (start 82.96 56.85) (end 82.96 49.95) (width 0.5) (layer "F.Cu") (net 1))
 (segment (start 82.96 71.51) (end 86.7375 75.2875) (width 0.5) (layer "F.Cu") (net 1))
 (segment (start 82.96 64.325) (end 82.96 71.51) (width 0.5) (layer "F.Cu") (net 1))
 (segment (start 85.55 50) (end 85.5 49.95) (width 0.5) (layer "F.Cu") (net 33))
 (segment (start 95.42 49) (end 91.425 49) (width 0.5) (layer "F.Cu") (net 33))
 (segment (start 90.425 50) (end 85.55 50) (width 0.5) (layer "F.Cu") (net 33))
 (segment (start 91.425 49) (end 90.425 50) (width 0.5) (layer "F.Cu") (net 33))
 (segment (start 89.225 56.85) (end 91.575 54.5) (width 0.5) (layer "F.Cu") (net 3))
 (segment (start 91.575 54.5) (end 95.42 54.5) (width 0.5) (layer "F.Cu") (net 3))
 (segment (start 85.5 56.85) (end 89.225 56.85) (width 0.5) (layer "F.Cu") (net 3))
 (segment (start 88.175 64.325) (end 92.5 60) (width 0.5) (layer "F.Cu") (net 5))
 (segment (start 85.5 64.325) (end 88.175 64.325) (width 0.5) (layer "F.Cu") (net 5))
 (segment (start 92.5 60) (end 95.42 60) (width 0.5) (layer "F.Cu") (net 5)))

